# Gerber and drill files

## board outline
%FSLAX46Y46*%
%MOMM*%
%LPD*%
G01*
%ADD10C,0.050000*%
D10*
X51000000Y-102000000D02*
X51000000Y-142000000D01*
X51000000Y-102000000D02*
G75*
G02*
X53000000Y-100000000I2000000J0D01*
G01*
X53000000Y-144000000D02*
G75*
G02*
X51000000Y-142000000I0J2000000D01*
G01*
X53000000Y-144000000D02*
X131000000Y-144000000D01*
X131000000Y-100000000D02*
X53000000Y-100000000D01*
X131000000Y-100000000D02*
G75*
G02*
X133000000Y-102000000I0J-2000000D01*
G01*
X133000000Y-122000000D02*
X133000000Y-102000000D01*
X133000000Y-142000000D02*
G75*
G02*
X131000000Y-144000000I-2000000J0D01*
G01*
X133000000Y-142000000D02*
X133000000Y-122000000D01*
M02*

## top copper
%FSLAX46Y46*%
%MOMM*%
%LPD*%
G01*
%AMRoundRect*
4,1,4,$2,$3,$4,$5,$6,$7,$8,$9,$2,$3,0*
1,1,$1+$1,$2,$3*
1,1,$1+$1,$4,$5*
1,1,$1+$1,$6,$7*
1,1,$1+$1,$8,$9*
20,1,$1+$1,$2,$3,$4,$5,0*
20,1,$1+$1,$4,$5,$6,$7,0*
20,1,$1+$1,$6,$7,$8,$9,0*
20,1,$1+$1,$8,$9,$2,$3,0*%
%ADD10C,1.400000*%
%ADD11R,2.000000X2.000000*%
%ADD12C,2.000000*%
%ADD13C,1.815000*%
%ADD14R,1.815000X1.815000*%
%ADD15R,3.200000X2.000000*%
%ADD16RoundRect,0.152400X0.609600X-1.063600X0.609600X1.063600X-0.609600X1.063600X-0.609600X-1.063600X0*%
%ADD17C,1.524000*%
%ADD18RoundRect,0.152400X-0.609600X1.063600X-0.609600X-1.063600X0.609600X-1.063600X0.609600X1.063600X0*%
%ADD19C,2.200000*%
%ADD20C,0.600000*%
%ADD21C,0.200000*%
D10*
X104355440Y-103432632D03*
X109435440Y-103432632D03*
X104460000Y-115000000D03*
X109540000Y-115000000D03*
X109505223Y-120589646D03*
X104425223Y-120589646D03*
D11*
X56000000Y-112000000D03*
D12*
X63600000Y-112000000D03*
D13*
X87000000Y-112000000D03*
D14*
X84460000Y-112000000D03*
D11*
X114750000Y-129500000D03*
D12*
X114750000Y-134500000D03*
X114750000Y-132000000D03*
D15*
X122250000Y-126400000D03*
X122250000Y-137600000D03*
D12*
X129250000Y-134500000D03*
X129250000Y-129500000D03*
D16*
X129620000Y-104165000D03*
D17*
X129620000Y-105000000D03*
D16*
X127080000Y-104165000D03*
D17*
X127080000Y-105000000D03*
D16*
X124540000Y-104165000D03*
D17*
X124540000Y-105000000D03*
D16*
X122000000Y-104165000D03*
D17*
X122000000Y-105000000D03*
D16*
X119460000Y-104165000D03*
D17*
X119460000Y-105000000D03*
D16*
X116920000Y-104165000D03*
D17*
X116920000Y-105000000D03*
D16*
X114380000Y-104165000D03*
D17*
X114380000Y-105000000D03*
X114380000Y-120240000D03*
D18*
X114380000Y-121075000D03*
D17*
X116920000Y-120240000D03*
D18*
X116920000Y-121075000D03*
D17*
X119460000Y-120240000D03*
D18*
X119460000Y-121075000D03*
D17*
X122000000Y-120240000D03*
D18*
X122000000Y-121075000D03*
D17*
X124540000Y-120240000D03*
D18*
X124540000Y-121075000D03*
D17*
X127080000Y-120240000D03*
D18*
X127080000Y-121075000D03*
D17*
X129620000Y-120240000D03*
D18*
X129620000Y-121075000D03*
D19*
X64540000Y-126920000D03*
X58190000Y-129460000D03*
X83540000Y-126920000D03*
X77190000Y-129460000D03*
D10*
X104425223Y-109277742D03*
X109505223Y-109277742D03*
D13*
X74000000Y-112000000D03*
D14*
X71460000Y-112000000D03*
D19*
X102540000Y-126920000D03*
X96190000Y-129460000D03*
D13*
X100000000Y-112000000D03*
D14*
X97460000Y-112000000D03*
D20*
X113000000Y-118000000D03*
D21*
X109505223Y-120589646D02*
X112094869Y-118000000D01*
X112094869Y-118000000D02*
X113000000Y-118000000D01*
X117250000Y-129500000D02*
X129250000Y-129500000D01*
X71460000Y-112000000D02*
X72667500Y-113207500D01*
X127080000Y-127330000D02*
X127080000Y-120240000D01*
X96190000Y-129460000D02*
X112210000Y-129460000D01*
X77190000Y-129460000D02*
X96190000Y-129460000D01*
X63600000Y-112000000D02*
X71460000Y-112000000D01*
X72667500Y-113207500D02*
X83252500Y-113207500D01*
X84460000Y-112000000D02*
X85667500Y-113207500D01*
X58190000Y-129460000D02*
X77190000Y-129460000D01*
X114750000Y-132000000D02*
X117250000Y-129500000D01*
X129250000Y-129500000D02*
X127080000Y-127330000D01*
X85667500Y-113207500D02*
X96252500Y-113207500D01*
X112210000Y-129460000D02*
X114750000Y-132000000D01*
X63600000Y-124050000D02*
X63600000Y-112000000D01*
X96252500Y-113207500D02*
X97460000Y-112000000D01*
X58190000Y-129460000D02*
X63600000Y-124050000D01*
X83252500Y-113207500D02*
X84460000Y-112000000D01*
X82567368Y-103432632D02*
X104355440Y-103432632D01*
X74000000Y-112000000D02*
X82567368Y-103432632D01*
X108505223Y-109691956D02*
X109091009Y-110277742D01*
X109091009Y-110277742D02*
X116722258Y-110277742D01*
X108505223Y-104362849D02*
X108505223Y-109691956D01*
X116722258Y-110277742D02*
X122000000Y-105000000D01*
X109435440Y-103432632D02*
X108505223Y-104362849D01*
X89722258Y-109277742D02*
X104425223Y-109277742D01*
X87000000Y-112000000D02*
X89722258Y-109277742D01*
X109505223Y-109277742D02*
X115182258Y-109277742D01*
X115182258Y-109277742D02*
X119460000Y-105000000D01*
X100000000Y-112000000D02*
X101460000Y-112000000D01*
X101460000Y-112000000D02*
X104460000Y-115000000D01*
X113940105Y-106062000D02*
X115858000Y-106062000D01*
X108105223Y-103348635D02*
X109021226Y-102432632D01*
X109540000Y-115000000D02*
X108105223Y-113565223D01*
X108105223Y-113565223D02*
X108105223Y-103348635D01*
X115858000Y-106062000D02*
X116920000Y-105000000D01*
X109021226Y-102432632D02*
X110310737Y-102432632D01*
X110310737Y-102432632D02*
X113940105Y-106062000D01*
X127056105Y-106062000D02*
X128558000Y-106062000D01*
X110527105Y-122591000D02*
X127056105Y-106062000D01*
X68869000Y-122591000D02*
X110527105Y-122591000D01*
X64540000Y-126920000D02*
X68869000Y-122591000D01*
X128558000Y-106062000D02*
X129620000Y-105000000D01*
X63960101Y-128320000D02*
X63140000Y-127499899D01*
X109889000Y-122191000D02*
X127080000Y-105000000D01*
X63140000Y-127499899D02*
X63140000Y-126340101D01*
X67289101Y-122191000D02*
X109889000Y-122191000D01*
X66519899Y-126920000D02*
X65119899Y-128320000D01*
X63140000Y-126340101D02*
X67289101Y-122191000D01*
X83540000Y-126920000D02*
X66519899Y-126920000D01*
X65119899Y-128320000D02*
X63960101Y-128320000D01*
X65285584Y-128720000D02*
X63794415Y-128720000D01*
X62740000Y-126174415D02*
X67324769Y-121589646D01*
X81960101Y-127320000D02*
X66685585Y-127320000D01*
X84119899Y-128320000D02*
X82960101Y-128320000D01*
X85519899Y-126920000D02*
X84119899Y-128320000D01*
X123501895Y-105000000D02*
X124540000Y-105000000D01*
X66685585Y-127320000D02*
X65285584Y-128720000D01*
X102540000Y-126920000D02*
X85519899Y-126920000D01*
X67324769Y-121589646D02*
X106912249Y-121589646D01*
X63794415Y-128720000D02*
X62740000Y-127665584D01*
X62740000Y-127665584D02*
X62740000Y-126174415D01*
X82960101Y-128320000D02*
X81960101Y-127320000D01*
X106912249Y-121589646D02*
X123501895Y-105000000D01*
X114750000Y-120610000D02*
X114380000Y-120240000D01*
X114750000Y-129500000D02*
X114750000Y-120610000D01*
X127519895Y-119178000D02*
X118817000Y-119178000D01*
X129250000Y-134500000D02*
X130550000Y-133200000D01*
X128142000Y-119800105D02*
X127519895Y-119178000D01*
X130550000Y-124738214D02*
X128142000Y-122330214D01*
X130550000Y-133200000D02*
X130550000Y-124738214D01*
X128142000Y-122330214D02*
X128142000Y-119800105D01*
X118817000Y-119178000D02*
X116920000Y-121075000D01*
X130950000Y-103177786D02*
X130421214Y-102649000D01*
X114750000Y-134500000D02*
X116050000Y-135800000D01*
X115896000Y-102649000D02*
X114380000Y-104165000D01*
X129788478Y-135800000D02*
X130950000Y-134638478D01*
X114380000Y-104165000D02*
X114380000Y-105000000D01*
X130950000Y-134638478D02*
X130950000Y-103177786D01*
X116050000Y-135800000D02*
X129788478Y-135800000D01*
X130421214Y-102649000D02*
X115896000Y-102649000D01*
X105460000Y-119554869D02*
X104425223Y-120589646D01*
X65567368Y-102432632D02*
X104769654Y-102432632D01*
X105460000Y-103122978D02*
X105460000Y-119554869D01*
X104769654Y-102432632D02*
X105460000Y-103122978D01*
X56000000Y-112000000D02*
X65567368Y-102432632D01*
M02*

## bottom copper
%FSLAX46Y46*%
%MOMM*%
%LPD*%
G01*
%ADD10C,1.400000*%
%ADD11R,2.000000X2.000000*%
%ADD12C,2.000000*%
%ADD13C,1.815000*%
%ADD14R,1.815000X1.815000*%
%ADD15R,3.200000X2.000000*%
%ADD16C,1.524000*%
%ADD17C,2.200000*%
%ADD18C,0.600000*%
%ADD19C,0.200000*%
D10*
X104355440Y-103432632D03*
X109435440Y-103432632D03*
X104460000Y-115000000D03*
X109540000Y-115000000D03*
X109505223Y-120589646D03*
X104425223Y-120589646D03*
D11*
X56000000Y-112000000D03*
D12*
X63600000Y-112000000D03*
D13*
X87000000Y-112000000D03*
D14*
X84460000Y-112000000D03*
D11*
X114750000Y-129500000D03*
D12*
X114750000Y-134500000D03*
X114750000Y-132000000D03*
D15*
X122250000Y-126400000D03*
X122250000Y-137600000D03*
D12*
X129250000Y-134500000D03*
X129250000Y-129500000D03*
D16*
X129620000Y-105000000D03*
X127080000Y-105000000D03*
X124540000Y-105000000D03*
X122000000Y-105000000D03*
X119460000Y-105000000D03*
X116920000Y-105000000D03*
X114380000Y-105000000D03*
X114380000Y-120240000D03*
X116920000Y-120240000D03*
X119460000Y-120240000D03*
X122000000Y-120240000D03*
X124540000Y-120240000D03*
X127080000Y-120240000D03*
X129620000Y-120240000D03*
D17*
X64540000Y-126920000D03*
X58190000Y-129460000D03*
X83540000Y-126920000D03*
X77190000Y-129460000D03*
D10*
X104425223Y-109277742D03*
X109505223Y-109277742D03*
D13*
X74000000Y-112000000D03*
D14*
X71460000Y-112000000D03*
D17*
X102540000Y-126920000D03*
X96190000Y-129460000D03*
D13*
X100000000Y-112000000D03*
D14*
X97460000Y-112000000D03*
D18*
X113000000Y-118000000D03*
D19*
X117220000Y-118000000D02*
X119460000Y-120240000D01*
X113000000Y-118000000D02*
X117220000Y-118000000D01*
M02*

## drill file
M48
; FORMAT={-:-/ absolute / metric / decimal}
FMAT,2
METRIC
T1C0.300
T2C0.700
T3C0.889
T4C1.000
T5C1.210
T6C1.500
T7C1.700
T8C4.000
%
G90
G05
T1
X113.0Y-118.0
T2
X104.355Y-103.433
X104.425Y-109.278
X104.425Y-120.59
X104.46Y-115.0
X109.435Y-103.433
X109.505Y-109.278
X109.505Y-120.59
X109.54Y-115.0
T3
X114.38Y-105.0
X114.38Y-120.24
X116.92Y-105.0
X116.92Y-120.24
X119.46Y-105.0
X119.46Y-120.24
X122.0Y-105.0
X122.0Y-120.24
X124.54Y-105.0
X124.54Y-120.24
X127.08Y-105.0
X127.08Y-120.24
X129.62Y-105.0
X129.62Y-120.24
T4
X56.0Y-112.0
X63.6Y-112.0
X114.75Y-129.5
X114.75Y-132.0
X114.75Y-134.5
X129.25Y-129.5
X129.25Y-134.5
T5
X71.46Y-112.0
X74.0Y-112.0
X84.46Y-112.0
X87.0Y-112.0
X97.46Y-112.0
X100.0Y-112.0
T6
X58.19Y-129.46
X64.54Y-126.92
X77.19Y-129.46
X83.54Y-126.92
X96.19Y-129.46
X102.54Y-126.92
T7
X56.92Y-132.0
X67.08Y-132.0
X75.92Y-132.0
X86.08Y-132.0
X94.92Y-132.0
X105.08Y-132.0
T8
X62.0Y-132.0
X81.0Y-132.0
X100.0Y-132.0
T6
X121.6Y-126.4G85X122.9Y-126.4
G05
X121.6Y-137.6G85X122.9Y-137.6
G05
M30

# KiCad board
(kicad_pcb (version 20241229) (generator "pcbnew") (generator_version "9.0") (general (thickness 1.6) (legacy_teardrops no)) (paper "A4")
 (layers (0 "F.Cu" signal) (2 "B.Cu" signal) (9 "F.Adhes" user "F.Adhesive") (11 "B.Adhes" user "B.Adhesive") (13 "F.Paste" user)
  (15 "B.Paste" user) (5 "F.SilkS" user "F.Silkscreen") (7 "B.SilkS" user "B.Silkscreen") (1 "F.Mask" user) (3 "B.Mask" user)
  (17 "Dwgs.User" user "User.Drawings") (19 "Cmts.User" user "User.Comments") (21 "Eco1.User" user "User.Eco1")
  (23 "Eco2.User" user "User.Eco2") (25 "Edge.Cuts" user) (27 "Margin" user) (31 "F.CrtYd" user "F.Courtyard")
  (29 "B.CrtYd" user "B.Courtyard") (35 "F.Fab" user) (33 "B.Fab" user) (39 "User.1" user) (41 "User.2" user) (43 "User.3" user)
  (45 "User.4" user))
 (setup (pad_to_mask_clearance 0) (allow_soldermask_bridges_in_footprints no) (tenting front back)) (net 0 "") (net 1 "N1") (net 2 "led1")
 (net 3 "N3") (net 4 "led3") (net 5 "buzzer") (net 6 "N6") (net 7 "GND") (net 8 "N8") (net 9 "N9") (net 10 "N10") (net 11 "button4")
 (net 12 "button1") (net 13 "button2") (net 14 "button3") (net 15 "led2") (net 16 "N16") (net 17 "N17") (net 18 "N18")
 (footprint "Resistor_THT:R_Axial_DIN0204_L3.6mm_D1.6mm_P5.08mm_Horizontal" (layer "F.Cu") (at 104.35544 103.432632)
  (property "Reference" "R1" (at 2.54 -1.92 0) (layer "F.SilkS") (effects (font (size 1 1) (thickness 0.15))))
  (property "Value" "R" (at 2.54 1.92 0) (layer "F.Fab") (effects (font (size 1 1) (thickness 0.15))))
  (pad "1" thru_hole circle (at 0 0) (size 1.4 1.4) (drill 0.7) (layers "*.Cu" "*.Mask") (remove_unused_layers no) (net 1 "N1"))
  (pad "2" thru_hole circle (at 5.08 0) (size 1.4 1.4) (drill 0.7) (layers "*.Cu" "*.Mask") (remove_unused_layers no) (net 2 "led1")))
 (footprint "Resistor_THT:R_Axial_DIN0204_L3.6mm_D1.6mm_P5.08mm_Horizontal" (layer "F.Cu") (at 104.46 115)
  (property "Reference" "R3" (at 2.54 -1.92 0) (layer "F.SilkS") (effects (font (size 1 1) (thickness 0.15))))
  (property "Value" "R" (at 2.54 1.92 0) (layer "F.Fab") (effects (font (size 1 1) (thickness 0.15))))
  (pad "1" thru_hole circle (at 0 0) (size 1.4 1.4) (drill 0.7) (layers "*.Cu" "*.Mask") (remove_unused_layers no) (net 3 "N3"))
  (pad "2" thru_hole circle (at 5.08 0) (size 1.4 1.4) (drill 0.7) (layers "*.Cu" "*.Mask") (remove_unused_layers no) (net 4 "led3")))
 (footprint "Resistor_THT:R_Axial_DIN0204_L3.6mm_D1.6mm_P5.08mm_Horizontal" (layer "F.Cu") (at 109.505223 120.589646 180)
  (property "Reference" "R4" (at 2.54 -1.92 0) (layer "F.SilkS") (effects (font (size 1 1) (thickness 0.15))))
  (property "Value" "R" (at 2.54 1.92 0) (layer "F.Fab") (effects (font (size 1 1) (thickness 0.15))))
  (pad "1" thru_hole circle (at 0 0 180) (size 1.4 1.4) (drill 0.7) (layers "*.Cu" "*.Mask") (remove_unused_layers no) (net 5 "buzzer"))
  (pad "2" thru_hole circle (at 5.08 0 180) (size 1.4 1.4) (drill 0.7) (layers "*.Cu" "*.Mask") (remove_unused_layers no) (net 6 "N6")))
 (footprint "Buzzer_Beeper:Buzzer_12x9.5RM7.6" (layer "F.Cu") (at 56 112)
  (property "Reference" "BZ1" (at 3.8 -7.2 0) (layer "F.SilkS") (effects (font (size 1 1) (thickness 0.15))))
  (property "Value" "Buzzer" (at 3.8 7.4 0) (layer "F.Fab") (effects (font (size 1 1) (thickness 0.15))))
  (pad "1" thru_hole rect (at 0 0) (size 2 2) (drill 1) (layers "*.Cu" "*.Mask") (remove_unused_layers no) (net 6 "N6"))
  (pad "2" thru_hole circle (at 7.6 0) (size 2 2) (drill 1) (layers "*.Cu" "*.Mask") (remove_unused_layers no) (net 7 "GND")))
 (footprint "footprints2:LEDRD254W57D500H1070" (layer "F.Cu") (at 85.73 112)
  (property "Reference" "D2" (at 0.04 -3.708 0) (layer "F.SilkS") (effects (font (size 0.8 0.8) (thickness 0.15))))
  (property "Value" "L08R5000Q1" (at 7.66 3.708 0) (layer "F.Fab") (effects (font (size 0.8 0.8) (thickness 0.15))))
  (pad "A" thru_hole circle (at 1.27 0) (size 1.815 1.815) (drill 1.21) (layers "*.Cu" "*.Mask") (remove_unused_layers no) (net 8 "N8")
   (solder_mask_margin 0.102))
  (pad "C" thru_hole rect (at -1.27 0) (size 1.815 1.815) (drill 1.21) (layers "*.Cu" "*.Mask") (remove_unused_layers no) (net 7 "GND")
   (solder_mask_margin 0.102)))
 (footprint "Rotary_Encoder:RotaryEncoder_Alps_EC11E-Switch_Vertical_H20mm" (layer "F.Cu") (at 114.75 129.5)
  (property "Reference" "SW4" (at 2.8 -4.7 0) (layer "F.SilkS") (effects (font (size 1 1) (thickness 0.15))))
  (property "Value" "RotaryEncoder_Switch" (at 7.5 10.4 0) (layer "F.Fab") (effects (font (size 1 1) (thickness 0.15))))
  (pad "A" thru_hole rect (at 0 0) (size 2 2) (drill 1) (layers "*.Cu" "*.Mask") (remove_unused_layers no) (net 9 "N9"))
  (pad "B" thru_hole circle (at 0 5) (size 2 2) (drill 1) (layers "*.Cu" "*.Mask") (remove_unused_layers no) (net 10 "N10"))
  (pad "C" thru_hole circle (at 0 2.5) (size 2 2) (drill 1) (layers "*.Cu" "*.Mask") (remove_unused_layers no) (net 7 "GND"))
  (pad "MP" thru_hole rect (at 7.5 -3.1) (size 3.2 2) (drill oval 2.8 1.5) (layers "*.Cu" "*.Mask") (remove_unused_layers no))
  (pad "MP" thru_hole rect (at 7.5 8.1) (size 3.2 2) (drill oval 2.8 1.5) (layers "*.Cu" "*.Mask") (remove_unused_layers no))
  (pad "S1" thru_hole circle (at 14.5 5) (size 2 2) (drill 1) (layers "*.Cu" "*.Mask") (remove_unused_layers no) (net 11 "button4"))
  (pad "S2" thru_hole circle (at 14.5 0) (size 2 2) (drill 1) (layers "*.Cu" "*.Mask") (remove_unused_layers no) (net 7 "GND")))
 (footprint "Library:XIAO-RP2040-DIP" (layer "F.Cu") (at 122 112.62)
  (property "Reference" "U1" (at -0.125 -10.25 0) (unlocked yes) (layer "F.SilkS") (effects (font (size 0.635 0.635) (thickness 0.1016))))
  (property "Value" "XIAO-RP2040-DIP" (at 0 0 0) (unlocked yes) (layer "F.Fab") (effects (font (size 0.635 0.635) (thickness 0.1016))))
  (pad "1" smd roundrect (at 7.62 -8.455 90) (size 2.432 1.524) (layers "F.Cu" "F.Mask") (roundrect_rratio 0.1) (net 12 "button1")
   (thermal_bridge_angle 45))
  (pad "1" thru_hole circle (at 7.62 -7.62 90) (size 1.524 1.524) (drill 0.889) (layers "*.Cu" "*.Mask") (remove_unused_layers no)
   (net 12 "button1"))
  (pad "2" smd roundrect (at 5.08 -8.455 90) (size 2.432 1.524) (layers "F.Cu" "F.Mask") (roundrect_rratio 0.1) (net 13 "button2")
   (thermal_bridge_angle 45))
  (pad "2" thru_hole circle (at 5.08 -7.62 90) (size 1.524 1.524) (drill 0.889) (layers "*.Cu" "*.Mask") (remove_unused_layers no)
   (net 13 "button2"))
  (pad "3" smd roundrect (at 2.54 -8.455 90) (size 2.432 1.524) (layers "F.Cu" "F.Mask") (roundrect_rratio 0.1) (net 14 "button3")
   (thermal_bridge_angle 45))
  (pad "3" thru_hole circle (at 2.54 -7.62 90) (size 1.524 1.524) (drill 0.889) (layers "*.Cu" "*.Mask") (remove_unused_layers no)
   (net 14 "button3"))
  (pad "4" smd roundrect (at 0 -8.455 90) (size 2.432 1.524) (layers "F.Cu" "F.Mask") (roundrect_rratio 0.1) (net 2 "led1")
   (thermal_bridge_angle 45))
  (pad "4" thru_hole circle (at 0 -7.62 90) (size 1.524 1.524) (drill 0.889) (layers "*.Cu" "*.Mask") (remove_unused_layers no)
   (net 2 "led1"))
  (pad "5" smd roundrect (at -2.54 -8.455 90) (size 2.432 1.524) (layers "F.Cu" "F.Mask") (roundrect_rratio 0.1) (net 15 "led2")
   (thermal_bridge_angle 45))
  (pad "5" thru_hole circle (at -2.54 -7.62 90) (size 1.524 1.524) (drill 0.889) (layers "*.Cu" "*.Mask") (remove_unused_layers no)
   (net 15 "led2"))
  (pad "6" smd roundrect (at -5.08 -8.455 90) (size 2.432 1.524) (layers "F.Cu" "F.Mask") (roundrect_rratio 0.1) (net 4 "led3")
   (thermal_bridge_angle 45))
  (pad "6" thru_hole circle (at -5.08 -7.62 90) (size 1.524 1.524) (drill 0.889) (layers "*.Cu" "*.Mask") (remove_unused_layers no)
   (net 4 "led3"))
  (pad "7" smd roundrect (at -7.62 -8.455 90) (size 2.432 1.524) (layers "F.Cu" "F.Mask") (roundrect_rratio 0.1) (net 10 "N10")
   (thermal_bridge_angle 45))
  (pad "7" thru_hole circle (at -7.62 -7.62 90) (size 1.524 1.524) (drill 0.889) (layers "*.Cu" "*.Mask") (remove_unused_layers no)
   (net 10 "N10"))
  (pad "8" thru_hole circle (at -7.62 7.62 270) (size 1.524 1.524) (drill 0.889) (layers "*.Cu" "*.Mask") (remove_unused_layers no)
   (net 9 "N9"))
  (pad "8" smd roundrect (at -7.62 8.455 270) (size 2.432 1.524) (layers "F.Cu" "F.Mask") (roundrect_rratio 0.1) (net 9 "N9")
   (thermal_bridge_angle 45))
  (pad "9" thru_hole circle (at -5.08 7.62 270) (size 1.524 1.524) (drill 0.889) (layers "*.Cu" "*.Mask") (remove_unused_layers no)
   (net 11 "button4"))
  (pad "9" smd roundrect (at -5.08 8.455 270) (size 2.432 1.524) (layers "F.Cu" "F.Mask") (roundrect_rratio 0.1) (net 11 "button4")
   (thermal_bridge_angle 45))
  (pad "10" thru_hole circle (at -2.54 7.62 270) (size 1.524 1.524) (drill 0.889) (layers "*.Cu" "*.Mask") (remove_unused_layers no)
   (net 5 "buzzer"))
  (pad "10" smd roundrect (at -2.54 8.455 270) (size 2.432 1.524) (layers "F.Cu" "F.Mask") (roundrect_rratio 0.1) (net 5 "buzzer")
   (thermal_bridge_angle 45))
  (pad "11" thru_hole circle (at 0 7.62 270) (size 1.524 1.524) (drill 0.889) (layers "*.Cu" "*.Mask") (remove_unused_layers no)
   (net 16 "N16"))
  (pad "11" smd roundrect (at 0 8.455 270) (size 2.432 1.524) (layers "F.Cu" "F.Mask") (roundrect_rratio 0.1) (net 16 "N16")
   (thermal_bridge_angle 45))
  (pad "12" thru_hole circle (at 2.54 7.62 270) (size 1.524 1.524) (drill 0.889) (layers "*.Cu" "*.Mask") (remove_unused_layers no)
   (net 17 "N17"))
  (pad "12" smd roundrect (at 2.54 8.455 270) (size 2.432 1.524) (layers "F.Cu" "F.Mask") (roundrect_rratio 0.1) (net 17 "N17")
   (thermal_bridge_angle 45))
  (pad "13" thru_hole circle (at 5.08 7.62 270) (size 1.524 1.524) (drill 0.889) (layers "*.Cu" "*.Mask") (remove_unused_layers no)
   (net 7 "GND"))
  (pad "13" smd roundrect (at 5.08 8.455 270) (size 2.432 1.524) (layers "F.Cu" "F.Mask") (roundrect_rratio 0.1) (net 7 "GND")
   (thermal_bridge_angle 45))
  (pad "14" thru_hole circle (at 7.62 7.62 270) (size 1.524 1.524) (drill 0.889) (layers "*.Cu" "*.Mask") (remove_unused_layers no)
   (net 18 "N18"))
  (pad "14" smd roundrect (at 7.62 8.455 270) (size 2.432 1.524) (layers "F.Cu" "F.Mask") (roundrect_rratio 0.1) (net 18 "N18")
   (thermal_bridge_angle 45)))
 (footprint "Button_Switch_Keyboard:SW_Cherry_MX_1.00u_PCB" (layer "F.Cu") (at 64.54 126.92)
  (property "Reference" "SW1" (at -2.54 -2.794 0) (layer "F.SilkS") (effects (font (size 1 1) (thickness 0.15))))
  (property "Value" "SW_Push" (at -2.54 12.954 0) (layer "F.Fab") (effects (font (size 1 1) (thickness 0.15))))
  (pad "" np_thru_hole circle (at -7.62 5.08) (size 1.7 1.7) (drill 1.7) (layers "*.Cu" "*.Mask"))
  (pad "" np_thru_hole circle (at -2.54 5.08) (size 4 4) (drill 4) (layers "*.Cu" "*.Mask"))
  (pad "" np_thru_hole circle (at 2.54 5.08) (size 1.7 1.7) (drill 1.7) (layers "*.Cu" "*.Mask"))
  (pad "1" thru_hole circle (at 0 0) (size 2.2 2.2) (drill 1.5) (layers "*.Cu" "*.Mask") (remove_unused_layers no) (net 12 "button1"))
  (pad "2" thru_hole circle (at -6.35 2.54) (size 2.2 2.2) (drill 1.5) (layers "*.Cu" "*.Mask") (remove_unused_layers no) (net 7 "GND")))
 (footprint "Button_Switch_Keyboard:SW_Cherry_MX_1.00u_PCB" (layer "F.Cu") (at 83.54 126.92)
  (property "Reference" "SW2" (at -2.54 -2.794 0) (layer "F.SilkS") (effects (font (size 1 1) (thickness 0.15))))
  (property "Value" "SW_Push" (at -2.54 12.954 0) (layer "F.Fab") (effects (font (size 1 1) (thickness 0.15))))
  (pad "" np_thru_hole circle (at -7.62 5.08) (size 1.7 1.7) (drill 1.7) (layers "*.Cu" "*.Mask"))
  (pad "" np_thru_hole circle (at -2.54 5.08) (size 4 4) (drill 4) (layers "*.Cu" "*.Mask"))
  (pad "" np_thru_hole circle (at 2.54 5.08) (size 1.7 1.7) (drill 1.7) (layers "*.Cu" "*.Mask"))
  (pad "1" thru_hole circle (at 0 0) (size 2.2 2.2) (drill 1.5) (layers "*.Cu" "*.Mask") (remove_unused_layers no) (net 13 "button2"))
  (pad "2" thru_hole circle (at -6.35 2.54) (size 2.2 2.2) (drill 1.5) (layers "*.Cu" "*.Mask") (remove_unused_layers no) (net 7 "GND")))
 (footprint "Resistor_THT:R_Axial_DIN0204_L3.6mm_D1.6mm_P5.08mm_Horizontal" (layer "F.Cu") (at 104.425223 109.277742)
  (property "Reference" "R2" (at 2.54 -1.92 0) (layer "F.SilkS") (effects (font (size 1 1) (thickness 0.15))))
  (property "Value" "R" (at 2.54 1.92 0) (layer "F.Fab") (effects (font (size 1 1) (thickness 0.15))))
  (pad "1" thru_hole circle (at 0 0) (size 1.4 1.4) (drill 0.7) (layers "*.Cu" "*.Mask") (remove_unused_layers no) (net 8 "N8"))
  (pad "2" thru_hole circle (at 5.08 0) (size 1.4 1.4) (drill 0.7) (layers "*.Cu" "*.Mask") (remove_unused_layers no) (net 15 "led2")))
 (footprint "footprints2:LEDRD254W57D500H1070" (layer "F.Cu") (at 72.73 112)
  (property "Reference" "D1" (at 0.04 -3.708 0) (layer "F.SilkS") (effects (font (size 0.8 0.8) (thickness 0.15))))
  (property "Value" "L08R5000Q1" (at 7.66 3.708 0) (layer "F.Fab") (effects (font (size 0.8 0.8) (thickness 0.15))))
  (pad "A" thru_hole circle (at 1.27 0) (size 1.815 1.815) (drill 1.21) (layers "*.Cu" "*.Mask") (remove_unused_layers no) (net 1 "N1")
   (solder_mask_margin 0.102))
  (pad "C" thru_hole rect (at -1.27 0) (size 1.815 1.815) (drill 1.21) (layers "*.Cu" "*.Mask") (remove_unused_layers no) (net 7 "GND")
   (solder_mask_margin 0.102)))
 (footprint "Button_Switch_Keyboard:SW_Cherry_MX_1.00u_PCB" (layer "F.Cu") (at 102.54 126.92)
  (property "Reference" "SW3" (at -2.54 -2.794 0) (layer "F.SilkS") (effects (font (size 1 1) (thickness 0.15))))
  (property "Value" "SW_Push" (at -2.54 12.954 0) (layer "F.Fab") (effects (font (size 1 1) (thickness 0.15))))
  (pad "" np_thru_hole circle (at -7.62 5.08) (size 1.7 1.7) (drill 1.7) (layers "*.Cu" "*.Mask"))
  (pad "" np_thru_hole circle (at -2.54 5.08) (size 4 4) (drill 4) (layers "*.Cu" "*.Mask"))
  (pad "" np_thru_hole circle (at 2.54 5.08) (size 1.7 1.7) (drill 1.7) (layers "*.Cu" "*.Mask"))
  (pad "1" thru_hole circle (at 0 0) (size 2.2 2.2) (drill 1.5) (layers "*.Cu" "*.Mask") (remove_unused_layers no) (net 14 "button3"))
  (pad "2" thru_hole circle (at -6.35 2.54) (size 2.2 2.2) (drill 1.5) (layers "*.Cu" "*.Mask") (remove_unused_layers no) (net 7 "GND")))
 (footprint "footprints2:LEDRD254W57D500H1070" (layer "F.Cu") (at 98.73 112)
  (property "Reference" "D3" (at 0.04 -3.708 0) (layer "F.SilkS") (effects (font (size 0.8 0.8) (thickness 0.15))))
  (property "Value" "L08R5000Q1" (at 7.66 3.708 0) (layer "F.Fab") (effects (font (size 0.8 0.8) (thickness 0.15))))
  (pad "A" thru_hole circle (at 1.27 0) (size 1.815 1.815) (drill 1.21) (layers "*.Cu" "*.Mask") (remove_unused_layers no) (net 3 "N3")
   (solder_mask_margin 0.102))
  (pad "C" thru_hole rect (at -1.27 0) (size 1.815 1.815) (drill 1.21) (layers "*.Cu" "*.Mask") (remove_unused_layers no) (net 7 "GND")
   (solder_mask_margin 0.102)))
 (gr_line (start 51 102) (end 51 142) (stroke (width 0.05) (type default)) (layer "Edge.Cuts"))
 (gr_arc (start 51 102) (mid 51.585786 100.585786) (end 53 100) (stroke (width 0.05) (type default)) (layer "Edge.Cuts"))
 (gr_arc (start 53 144) (mid 51.585786 143.414214) (end 51 142) (stroke (width 0.05) (type default)) (layer "Edge.Cuts"))
 (gr_line (start 53 144) (end 131 144) (stroke (width 0.05) (type default)) (layer "Edge.Cuts"))
 (gr_line (start 131 100) (end 53 100) (stroke (width 0.05) (type default)) (layer "Edge.Cuts"))
 (gr_arc (start 131 100) (mid 132.414214 100.585786) (end 133 102) (stroke (width 0.05) (type default)) (layer "Edge.Cuts"))
 (gr_line (start 133 122) (end 133 102) (stroke (width 0.05) (type default)) (layer "Edge.Cuts"))
 (gr_arc (start 133 142) (mid 132.414214 143.414214) (end 131 144) (stroke (width 0.05) (type default)) (layer "Edge.Cuts"))
 (gr_line (start 133 142) (end 133 122) (stroke (width 0.05) (type default)) (layer "Edge.Cuts"))
 (segment (start 109.505223 120.589646) (end 112.094869 118) (width 0.2) (layer "F.Cu") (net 5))
 (segment (start 112.094869 118) (end 113 118) (width 0.2) (layer "F.Cu") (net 5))
 (via (at 113 118) (size 0.6) (drill 0.3) (layers "F.Cu" "B.Cu") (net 5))
 (segment (start 117.22 118) (end 119.46 120.24) (width 0.2) (layer "B.Cu") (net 5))
 (segment (start 113 118) (end 117.22 118) (width 0.2) (layer "B.Cu") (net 5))
 (segment (start 117.25 129.5) (end 129.25 129.5) (width 0.2) (layer "F.Cu") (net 7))
 (segment (start 71.46 112) (end 72.6675 113.2075) (width 0.2) (layer "F.Cu") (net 7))
 (segment (start 127.08 127.33) (end 127.08 120.24) (width 0.2) (layer "F.Cu") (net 7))
 (segment (start 96.19 129.46) (end 112.21 129.46) (width 0.2) (layer "F.Cu") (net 7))
 (segment (start 77.19 129.46) (end 96.19 129.46) (width 0.2) (layer "F.Cu") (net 7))
 (segment (start 63.6 112) (end 71.46 112) (width 0.2) (layer "F.Cu") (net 7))
 (segment (start 72.6675 113.2075) (end 83.2525 113.2075) (width 0.2) (layer "F.Cu") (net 7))
 (segment (start 84.46 112) (end 85.6675 113.2075) (width 0.2) (layer "F.Cu") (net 7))
 (segment (start 58.19 129.46) (end 77.19 129.46) (width 0.2) (layer "F.Cu") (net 7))
 (segment (start 114.75 132) (end 117.25 129.5) (width 0.2) (layer "F.Cu") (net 7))
 (segment (start 129.25 129.5) (end 127.08 127.33) (width 0.2) (layer "F.Cu") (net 7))
 (segment (start 85.6675 113.2075) (end 96.2525 113.2075) (width 0.2) (layer "F.Cu") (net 7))
 (segment (start 112.21 129.46) (end 114.75 132) (width 0.2) (layer "F.Cu") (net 7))
 (segment (start 63.6 124.05) (end 63.6 112) (width 0.2) (layer "F.Cu") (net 7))
 (segment (start 96.2525 113.2075) (end 97.46 112) (width 0.2) (layer "F.Cu") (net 7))
 (segment (start 58.19 129.46) (end 63.6 124.05) (width 0.2) (layer "F.Cu") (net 7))
 (segment (start 83.2525 113.2075) (end 84.46 112) (width 0.2) (layer "F.Cu") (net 7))
 (segment (start 82.567368 103.432632) (end 104.35544 103.432632) (width 0.2) (layer "F.Cu") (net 1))
 (segment (start 74 112) (end 82.567368 103.432632) (width 0.2) (layer "F.Cu") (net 1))
 (segment (start 108.505223 109.691956) (end 109.091009 110.277742) (width 0.2) (layer "F.Cu") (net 2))
 (segment (start 109.091009 110.277742) (end 116.722258 110.277742) (width 0.2) (layer "F.Cu") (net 2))
 (segment (start 108.505223 104.362849) (end 108.505223 109.691956) (width 0.2) (layer "F.Cu") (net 2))
 (segment (start 116.722258 110.277742) (end 122 105) (width 0.2) (layer "F.Cu") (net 2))
 (segment (start 109.43544 103.432632) (end 108.505223 104.362849) (width 0.2) (layer "F.Cu") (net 2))
 (segment (start 89.722258 109.277742) (end 104.425223 109.277742) (width 0.2) (layer "F.Cu") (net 8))
 (segment (start 87 112) (end 89.722258 109.277742) (width 0.2) (layer "F.Cu") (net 8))
 (segment (start 109.505223 109.277742) (end 115.182258 109.277742) (width 0.2) (layer "F.Cu") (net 15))
 (segment (start 115.182258 109.277742) (end 119.46 105) (width 0.2) (layer "F.Cu") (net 15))
 (segment (start 100 112) (end 101.46 112) (width 0.2) (layer "F.Cu") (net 3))
 (segment (start 101.46 112) (end 104.46 115) (width 0.2) (layer "F.Cu") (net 3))
 (segment (start 113.940105 106.062) (end 115.858 106.062) (width 0.2) (layer "F.Cu") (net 4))
 (segment (start 108.105223 103.348635) (end 109.021226 102.432632) (width 0.2) (layer "F.Cu") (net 4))
 (segment (start 109.54 115) (end 108.105223 113.565223) (width 0.2) (layer "F.Cu") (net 4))
 (segment (start 108.105223 113.565223) (end 108.105223 103.348635) (width 0.2) (layer "F.Cu") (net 4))
 (segment (start 115.858 106.062) (end 116.92 105) (width 0.2) (layer "F.Cu") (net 4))
 (segment (start 109.021226 102.432632) (end 110.310737 102.432632) (width 0.2) (layer "F.Cu") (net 4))
 (segment (start 110.310737 102.432632) (end 113.940105 106.062) (width 0.2) (layer "F.Cu") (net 4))
 (segment (start 127.056105 106.062) (end 128.558 106.062) (width 0.2) (layer "F.Cu") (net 12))
 (segment (start 110.527105 122.591) (end 127.056105 106.062) (width 0.2) (layer "F.Cu") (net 12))
 (segment (start 68.869 122.591) (end 110.527105 122.591) (width 0.2) (layer "F.Cu") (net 12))
 (segment (start 64.54 126.92) (end 68.869 122.591) (width 0.2) (layer "F.Cu") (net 12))
 (segment (start 128.558 106.062) (end 129.62 105) (width 0.2) (layer "F.Cu") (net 12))
 (segment (start 63.960101 128.32) (end 63.14 127.499899) (width 0.2) (layer "F.Cu") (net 13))
 (segment (start 109.889 122.191) (end 127.08 105) (width 0.2) (layer "F.Cu") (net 13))
 (segment (start 63.14 127.499899) (end 63.14 126.340101) (width 0.2) (layer "F.Cu") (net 13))
 (segment (start 67.289101 122.191) (end 109.889 122.191) (width 0.2) (layer "F.Cu") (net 13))
 (segment (start 66.519899 126.92) (end 65.119899 128.32) (width 0.2) (layer "F.Cu") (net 13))
 (segment (start 63.14 126.340101) (end 67.289101 122.191) (width 0.2) (layer "F.Cu") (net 13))
 (segment (start 83.54 126.92) (end 66.519899 126.92) (width 0.2) (layer "F.Cu") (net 13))
 (segment (start 65.119899 128.32) (end 63.960101 128.32) (width 0.2) (layer "F.Cu") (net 13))
 (segment (start 65.285584 128.72) (end 63.794415 128.72) (width 0.2) (layer "F.Cu") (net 14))
 (segment (start 62.74 126.174415) (end 67.324769 121.589646) (width 0.2) (layer "F.Cu") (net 14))
 (segment (start 81.960101 127.32) (end 66.685585 127.32) (width 0.2) (layer "F.Cu") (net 14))
 (segment (start 84.119899 128.32) (end 82.960101 128.32) (width 0.2) (layer "F.Cu") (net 14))
 (segment (start 85.519899 126.92) (end 84.119899 128.32) (width 0.2) (layer "F.Cu") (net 14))
 (segment (start 123.501895 105) (end 124.54 105) (width 0.2) (layer "F.Cu") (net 14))
 (segment (start 66.685585 127.32) (end 65.285584 128.72) (width 0.2) (layer "F.Cu") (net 14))
 (segment (start 102.54 126.92) (end 85.519899 126.92) (width 0.2) (layer "F.Cu") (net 14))
 (segment (start 67.324769 121.589646) (end 106.912249 121.589646) (width 0.2) (layer "F.Cu") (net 14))
 (segment (start 63.794415 128.72) (end 62.74 127.665584) (width 0.2) (layer "F.Cu") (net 14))
 (segment (start 62.74 127.665584) (end 62.74 126.174415) (width 0.2) (layer "F.Cu") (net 14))
 (segment (start 82.960101 128.32) (end 81.960101 127.32) (width 0.2) (layer "F.Cu") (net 14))
 (segment (start 106.912249 121.589646) (end 123.501895 105) (width 0.2) (layer "F.Cu") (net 14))
 (segment (start 114.75 120.61) (end 114.38 120.24) (width 0.2) (layer "F.Cu") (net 9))
 (segment (start 114.75 129.5) (end 114.75 120.61) (width 0.2) (layer "F.Cu") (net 9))
 (segment (start 127.519895 119.178) (end 118.817 119.178) (width 0.2) (layer "F.Cu") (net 11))
 (segment (start 129.25 134.5) (end 130.55 133.2) (width 0.2) (layer "F.Cu") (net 11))
 (segment (start 128.142 119.800105) (end 127.519895 119.178) (width 0.2) (layer "F.Cu") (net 11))
 (segment (start 130.55 124.738214) (end 128.142 122.330214) (width 0.2) (layer "F.Cu") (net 11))
 (segment (start 130.55 133.2) (end 130.55 124.738214) (width 0.2) (layer "F.Cu") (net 11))
 (segment (start 128.142 122.330214) (end 128.142 119.800105) (width 0.2) (layer "F.Cu") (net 11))
 (segment (start 118.817 119.178) (end 116.92 121.075) (width 0.2) (layer "F.Cu") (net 11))
 (segment (start 130.95 103.177786) (end 130.421214 102.649) (width 0.2) (layer "F.Cu") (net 10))
 (segment (start 114.75 134.5) (end 116.05 135.8) (width 0.2) (layer "F.Cu") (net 10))
 (segment (start 115.896 102.649) (end 114.38 104.165) (width 0.2) (layer "F.Cu") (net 10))
 (segment (start 129.788478 135.8) (end 130.95 134.638478) (width 0.2) (layer "F.Cu") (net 10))
 (segment (start 114.38 104.165) (end 114.38 105) (width 0.2) (layer "F.Cu") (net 10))
 (segment (start 130.95 134.638478) (end 130.95 103.177786) (width 0.2) (layer "F.Cu") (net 10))
 (segment (start 116.05 135.8) (end 129.788478 135.8) (width 0.2) (layer "F.Cu") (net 10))
 (segment (start 130.421214 102.649) (end 115.896 102.649) (width 0.2) (layer "F.Cu") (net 10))
 (segment (start 105.46 119.554869) (end 104.425223 120.589646) (width 0.2) (layer "F.Cu") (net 6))
 (segment (start 65.567368 102.432632) (end 104.769654 102.432632) (width 0.2) (layer "F.Cu") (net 6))
 (segment (start 105.46 103.122978) (end 105.46 119.554869) (width 0.2) (layer "F.Cu") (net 6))
 (segment (start 104.769654 102.432632) (end 105.46 103.122978) (width 0.2) (layer "F.Cu") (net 6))
 (segment (start 56 112) (end 65.567368 102.432632) (width 0.2) (layer "F.Cu") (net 6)))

